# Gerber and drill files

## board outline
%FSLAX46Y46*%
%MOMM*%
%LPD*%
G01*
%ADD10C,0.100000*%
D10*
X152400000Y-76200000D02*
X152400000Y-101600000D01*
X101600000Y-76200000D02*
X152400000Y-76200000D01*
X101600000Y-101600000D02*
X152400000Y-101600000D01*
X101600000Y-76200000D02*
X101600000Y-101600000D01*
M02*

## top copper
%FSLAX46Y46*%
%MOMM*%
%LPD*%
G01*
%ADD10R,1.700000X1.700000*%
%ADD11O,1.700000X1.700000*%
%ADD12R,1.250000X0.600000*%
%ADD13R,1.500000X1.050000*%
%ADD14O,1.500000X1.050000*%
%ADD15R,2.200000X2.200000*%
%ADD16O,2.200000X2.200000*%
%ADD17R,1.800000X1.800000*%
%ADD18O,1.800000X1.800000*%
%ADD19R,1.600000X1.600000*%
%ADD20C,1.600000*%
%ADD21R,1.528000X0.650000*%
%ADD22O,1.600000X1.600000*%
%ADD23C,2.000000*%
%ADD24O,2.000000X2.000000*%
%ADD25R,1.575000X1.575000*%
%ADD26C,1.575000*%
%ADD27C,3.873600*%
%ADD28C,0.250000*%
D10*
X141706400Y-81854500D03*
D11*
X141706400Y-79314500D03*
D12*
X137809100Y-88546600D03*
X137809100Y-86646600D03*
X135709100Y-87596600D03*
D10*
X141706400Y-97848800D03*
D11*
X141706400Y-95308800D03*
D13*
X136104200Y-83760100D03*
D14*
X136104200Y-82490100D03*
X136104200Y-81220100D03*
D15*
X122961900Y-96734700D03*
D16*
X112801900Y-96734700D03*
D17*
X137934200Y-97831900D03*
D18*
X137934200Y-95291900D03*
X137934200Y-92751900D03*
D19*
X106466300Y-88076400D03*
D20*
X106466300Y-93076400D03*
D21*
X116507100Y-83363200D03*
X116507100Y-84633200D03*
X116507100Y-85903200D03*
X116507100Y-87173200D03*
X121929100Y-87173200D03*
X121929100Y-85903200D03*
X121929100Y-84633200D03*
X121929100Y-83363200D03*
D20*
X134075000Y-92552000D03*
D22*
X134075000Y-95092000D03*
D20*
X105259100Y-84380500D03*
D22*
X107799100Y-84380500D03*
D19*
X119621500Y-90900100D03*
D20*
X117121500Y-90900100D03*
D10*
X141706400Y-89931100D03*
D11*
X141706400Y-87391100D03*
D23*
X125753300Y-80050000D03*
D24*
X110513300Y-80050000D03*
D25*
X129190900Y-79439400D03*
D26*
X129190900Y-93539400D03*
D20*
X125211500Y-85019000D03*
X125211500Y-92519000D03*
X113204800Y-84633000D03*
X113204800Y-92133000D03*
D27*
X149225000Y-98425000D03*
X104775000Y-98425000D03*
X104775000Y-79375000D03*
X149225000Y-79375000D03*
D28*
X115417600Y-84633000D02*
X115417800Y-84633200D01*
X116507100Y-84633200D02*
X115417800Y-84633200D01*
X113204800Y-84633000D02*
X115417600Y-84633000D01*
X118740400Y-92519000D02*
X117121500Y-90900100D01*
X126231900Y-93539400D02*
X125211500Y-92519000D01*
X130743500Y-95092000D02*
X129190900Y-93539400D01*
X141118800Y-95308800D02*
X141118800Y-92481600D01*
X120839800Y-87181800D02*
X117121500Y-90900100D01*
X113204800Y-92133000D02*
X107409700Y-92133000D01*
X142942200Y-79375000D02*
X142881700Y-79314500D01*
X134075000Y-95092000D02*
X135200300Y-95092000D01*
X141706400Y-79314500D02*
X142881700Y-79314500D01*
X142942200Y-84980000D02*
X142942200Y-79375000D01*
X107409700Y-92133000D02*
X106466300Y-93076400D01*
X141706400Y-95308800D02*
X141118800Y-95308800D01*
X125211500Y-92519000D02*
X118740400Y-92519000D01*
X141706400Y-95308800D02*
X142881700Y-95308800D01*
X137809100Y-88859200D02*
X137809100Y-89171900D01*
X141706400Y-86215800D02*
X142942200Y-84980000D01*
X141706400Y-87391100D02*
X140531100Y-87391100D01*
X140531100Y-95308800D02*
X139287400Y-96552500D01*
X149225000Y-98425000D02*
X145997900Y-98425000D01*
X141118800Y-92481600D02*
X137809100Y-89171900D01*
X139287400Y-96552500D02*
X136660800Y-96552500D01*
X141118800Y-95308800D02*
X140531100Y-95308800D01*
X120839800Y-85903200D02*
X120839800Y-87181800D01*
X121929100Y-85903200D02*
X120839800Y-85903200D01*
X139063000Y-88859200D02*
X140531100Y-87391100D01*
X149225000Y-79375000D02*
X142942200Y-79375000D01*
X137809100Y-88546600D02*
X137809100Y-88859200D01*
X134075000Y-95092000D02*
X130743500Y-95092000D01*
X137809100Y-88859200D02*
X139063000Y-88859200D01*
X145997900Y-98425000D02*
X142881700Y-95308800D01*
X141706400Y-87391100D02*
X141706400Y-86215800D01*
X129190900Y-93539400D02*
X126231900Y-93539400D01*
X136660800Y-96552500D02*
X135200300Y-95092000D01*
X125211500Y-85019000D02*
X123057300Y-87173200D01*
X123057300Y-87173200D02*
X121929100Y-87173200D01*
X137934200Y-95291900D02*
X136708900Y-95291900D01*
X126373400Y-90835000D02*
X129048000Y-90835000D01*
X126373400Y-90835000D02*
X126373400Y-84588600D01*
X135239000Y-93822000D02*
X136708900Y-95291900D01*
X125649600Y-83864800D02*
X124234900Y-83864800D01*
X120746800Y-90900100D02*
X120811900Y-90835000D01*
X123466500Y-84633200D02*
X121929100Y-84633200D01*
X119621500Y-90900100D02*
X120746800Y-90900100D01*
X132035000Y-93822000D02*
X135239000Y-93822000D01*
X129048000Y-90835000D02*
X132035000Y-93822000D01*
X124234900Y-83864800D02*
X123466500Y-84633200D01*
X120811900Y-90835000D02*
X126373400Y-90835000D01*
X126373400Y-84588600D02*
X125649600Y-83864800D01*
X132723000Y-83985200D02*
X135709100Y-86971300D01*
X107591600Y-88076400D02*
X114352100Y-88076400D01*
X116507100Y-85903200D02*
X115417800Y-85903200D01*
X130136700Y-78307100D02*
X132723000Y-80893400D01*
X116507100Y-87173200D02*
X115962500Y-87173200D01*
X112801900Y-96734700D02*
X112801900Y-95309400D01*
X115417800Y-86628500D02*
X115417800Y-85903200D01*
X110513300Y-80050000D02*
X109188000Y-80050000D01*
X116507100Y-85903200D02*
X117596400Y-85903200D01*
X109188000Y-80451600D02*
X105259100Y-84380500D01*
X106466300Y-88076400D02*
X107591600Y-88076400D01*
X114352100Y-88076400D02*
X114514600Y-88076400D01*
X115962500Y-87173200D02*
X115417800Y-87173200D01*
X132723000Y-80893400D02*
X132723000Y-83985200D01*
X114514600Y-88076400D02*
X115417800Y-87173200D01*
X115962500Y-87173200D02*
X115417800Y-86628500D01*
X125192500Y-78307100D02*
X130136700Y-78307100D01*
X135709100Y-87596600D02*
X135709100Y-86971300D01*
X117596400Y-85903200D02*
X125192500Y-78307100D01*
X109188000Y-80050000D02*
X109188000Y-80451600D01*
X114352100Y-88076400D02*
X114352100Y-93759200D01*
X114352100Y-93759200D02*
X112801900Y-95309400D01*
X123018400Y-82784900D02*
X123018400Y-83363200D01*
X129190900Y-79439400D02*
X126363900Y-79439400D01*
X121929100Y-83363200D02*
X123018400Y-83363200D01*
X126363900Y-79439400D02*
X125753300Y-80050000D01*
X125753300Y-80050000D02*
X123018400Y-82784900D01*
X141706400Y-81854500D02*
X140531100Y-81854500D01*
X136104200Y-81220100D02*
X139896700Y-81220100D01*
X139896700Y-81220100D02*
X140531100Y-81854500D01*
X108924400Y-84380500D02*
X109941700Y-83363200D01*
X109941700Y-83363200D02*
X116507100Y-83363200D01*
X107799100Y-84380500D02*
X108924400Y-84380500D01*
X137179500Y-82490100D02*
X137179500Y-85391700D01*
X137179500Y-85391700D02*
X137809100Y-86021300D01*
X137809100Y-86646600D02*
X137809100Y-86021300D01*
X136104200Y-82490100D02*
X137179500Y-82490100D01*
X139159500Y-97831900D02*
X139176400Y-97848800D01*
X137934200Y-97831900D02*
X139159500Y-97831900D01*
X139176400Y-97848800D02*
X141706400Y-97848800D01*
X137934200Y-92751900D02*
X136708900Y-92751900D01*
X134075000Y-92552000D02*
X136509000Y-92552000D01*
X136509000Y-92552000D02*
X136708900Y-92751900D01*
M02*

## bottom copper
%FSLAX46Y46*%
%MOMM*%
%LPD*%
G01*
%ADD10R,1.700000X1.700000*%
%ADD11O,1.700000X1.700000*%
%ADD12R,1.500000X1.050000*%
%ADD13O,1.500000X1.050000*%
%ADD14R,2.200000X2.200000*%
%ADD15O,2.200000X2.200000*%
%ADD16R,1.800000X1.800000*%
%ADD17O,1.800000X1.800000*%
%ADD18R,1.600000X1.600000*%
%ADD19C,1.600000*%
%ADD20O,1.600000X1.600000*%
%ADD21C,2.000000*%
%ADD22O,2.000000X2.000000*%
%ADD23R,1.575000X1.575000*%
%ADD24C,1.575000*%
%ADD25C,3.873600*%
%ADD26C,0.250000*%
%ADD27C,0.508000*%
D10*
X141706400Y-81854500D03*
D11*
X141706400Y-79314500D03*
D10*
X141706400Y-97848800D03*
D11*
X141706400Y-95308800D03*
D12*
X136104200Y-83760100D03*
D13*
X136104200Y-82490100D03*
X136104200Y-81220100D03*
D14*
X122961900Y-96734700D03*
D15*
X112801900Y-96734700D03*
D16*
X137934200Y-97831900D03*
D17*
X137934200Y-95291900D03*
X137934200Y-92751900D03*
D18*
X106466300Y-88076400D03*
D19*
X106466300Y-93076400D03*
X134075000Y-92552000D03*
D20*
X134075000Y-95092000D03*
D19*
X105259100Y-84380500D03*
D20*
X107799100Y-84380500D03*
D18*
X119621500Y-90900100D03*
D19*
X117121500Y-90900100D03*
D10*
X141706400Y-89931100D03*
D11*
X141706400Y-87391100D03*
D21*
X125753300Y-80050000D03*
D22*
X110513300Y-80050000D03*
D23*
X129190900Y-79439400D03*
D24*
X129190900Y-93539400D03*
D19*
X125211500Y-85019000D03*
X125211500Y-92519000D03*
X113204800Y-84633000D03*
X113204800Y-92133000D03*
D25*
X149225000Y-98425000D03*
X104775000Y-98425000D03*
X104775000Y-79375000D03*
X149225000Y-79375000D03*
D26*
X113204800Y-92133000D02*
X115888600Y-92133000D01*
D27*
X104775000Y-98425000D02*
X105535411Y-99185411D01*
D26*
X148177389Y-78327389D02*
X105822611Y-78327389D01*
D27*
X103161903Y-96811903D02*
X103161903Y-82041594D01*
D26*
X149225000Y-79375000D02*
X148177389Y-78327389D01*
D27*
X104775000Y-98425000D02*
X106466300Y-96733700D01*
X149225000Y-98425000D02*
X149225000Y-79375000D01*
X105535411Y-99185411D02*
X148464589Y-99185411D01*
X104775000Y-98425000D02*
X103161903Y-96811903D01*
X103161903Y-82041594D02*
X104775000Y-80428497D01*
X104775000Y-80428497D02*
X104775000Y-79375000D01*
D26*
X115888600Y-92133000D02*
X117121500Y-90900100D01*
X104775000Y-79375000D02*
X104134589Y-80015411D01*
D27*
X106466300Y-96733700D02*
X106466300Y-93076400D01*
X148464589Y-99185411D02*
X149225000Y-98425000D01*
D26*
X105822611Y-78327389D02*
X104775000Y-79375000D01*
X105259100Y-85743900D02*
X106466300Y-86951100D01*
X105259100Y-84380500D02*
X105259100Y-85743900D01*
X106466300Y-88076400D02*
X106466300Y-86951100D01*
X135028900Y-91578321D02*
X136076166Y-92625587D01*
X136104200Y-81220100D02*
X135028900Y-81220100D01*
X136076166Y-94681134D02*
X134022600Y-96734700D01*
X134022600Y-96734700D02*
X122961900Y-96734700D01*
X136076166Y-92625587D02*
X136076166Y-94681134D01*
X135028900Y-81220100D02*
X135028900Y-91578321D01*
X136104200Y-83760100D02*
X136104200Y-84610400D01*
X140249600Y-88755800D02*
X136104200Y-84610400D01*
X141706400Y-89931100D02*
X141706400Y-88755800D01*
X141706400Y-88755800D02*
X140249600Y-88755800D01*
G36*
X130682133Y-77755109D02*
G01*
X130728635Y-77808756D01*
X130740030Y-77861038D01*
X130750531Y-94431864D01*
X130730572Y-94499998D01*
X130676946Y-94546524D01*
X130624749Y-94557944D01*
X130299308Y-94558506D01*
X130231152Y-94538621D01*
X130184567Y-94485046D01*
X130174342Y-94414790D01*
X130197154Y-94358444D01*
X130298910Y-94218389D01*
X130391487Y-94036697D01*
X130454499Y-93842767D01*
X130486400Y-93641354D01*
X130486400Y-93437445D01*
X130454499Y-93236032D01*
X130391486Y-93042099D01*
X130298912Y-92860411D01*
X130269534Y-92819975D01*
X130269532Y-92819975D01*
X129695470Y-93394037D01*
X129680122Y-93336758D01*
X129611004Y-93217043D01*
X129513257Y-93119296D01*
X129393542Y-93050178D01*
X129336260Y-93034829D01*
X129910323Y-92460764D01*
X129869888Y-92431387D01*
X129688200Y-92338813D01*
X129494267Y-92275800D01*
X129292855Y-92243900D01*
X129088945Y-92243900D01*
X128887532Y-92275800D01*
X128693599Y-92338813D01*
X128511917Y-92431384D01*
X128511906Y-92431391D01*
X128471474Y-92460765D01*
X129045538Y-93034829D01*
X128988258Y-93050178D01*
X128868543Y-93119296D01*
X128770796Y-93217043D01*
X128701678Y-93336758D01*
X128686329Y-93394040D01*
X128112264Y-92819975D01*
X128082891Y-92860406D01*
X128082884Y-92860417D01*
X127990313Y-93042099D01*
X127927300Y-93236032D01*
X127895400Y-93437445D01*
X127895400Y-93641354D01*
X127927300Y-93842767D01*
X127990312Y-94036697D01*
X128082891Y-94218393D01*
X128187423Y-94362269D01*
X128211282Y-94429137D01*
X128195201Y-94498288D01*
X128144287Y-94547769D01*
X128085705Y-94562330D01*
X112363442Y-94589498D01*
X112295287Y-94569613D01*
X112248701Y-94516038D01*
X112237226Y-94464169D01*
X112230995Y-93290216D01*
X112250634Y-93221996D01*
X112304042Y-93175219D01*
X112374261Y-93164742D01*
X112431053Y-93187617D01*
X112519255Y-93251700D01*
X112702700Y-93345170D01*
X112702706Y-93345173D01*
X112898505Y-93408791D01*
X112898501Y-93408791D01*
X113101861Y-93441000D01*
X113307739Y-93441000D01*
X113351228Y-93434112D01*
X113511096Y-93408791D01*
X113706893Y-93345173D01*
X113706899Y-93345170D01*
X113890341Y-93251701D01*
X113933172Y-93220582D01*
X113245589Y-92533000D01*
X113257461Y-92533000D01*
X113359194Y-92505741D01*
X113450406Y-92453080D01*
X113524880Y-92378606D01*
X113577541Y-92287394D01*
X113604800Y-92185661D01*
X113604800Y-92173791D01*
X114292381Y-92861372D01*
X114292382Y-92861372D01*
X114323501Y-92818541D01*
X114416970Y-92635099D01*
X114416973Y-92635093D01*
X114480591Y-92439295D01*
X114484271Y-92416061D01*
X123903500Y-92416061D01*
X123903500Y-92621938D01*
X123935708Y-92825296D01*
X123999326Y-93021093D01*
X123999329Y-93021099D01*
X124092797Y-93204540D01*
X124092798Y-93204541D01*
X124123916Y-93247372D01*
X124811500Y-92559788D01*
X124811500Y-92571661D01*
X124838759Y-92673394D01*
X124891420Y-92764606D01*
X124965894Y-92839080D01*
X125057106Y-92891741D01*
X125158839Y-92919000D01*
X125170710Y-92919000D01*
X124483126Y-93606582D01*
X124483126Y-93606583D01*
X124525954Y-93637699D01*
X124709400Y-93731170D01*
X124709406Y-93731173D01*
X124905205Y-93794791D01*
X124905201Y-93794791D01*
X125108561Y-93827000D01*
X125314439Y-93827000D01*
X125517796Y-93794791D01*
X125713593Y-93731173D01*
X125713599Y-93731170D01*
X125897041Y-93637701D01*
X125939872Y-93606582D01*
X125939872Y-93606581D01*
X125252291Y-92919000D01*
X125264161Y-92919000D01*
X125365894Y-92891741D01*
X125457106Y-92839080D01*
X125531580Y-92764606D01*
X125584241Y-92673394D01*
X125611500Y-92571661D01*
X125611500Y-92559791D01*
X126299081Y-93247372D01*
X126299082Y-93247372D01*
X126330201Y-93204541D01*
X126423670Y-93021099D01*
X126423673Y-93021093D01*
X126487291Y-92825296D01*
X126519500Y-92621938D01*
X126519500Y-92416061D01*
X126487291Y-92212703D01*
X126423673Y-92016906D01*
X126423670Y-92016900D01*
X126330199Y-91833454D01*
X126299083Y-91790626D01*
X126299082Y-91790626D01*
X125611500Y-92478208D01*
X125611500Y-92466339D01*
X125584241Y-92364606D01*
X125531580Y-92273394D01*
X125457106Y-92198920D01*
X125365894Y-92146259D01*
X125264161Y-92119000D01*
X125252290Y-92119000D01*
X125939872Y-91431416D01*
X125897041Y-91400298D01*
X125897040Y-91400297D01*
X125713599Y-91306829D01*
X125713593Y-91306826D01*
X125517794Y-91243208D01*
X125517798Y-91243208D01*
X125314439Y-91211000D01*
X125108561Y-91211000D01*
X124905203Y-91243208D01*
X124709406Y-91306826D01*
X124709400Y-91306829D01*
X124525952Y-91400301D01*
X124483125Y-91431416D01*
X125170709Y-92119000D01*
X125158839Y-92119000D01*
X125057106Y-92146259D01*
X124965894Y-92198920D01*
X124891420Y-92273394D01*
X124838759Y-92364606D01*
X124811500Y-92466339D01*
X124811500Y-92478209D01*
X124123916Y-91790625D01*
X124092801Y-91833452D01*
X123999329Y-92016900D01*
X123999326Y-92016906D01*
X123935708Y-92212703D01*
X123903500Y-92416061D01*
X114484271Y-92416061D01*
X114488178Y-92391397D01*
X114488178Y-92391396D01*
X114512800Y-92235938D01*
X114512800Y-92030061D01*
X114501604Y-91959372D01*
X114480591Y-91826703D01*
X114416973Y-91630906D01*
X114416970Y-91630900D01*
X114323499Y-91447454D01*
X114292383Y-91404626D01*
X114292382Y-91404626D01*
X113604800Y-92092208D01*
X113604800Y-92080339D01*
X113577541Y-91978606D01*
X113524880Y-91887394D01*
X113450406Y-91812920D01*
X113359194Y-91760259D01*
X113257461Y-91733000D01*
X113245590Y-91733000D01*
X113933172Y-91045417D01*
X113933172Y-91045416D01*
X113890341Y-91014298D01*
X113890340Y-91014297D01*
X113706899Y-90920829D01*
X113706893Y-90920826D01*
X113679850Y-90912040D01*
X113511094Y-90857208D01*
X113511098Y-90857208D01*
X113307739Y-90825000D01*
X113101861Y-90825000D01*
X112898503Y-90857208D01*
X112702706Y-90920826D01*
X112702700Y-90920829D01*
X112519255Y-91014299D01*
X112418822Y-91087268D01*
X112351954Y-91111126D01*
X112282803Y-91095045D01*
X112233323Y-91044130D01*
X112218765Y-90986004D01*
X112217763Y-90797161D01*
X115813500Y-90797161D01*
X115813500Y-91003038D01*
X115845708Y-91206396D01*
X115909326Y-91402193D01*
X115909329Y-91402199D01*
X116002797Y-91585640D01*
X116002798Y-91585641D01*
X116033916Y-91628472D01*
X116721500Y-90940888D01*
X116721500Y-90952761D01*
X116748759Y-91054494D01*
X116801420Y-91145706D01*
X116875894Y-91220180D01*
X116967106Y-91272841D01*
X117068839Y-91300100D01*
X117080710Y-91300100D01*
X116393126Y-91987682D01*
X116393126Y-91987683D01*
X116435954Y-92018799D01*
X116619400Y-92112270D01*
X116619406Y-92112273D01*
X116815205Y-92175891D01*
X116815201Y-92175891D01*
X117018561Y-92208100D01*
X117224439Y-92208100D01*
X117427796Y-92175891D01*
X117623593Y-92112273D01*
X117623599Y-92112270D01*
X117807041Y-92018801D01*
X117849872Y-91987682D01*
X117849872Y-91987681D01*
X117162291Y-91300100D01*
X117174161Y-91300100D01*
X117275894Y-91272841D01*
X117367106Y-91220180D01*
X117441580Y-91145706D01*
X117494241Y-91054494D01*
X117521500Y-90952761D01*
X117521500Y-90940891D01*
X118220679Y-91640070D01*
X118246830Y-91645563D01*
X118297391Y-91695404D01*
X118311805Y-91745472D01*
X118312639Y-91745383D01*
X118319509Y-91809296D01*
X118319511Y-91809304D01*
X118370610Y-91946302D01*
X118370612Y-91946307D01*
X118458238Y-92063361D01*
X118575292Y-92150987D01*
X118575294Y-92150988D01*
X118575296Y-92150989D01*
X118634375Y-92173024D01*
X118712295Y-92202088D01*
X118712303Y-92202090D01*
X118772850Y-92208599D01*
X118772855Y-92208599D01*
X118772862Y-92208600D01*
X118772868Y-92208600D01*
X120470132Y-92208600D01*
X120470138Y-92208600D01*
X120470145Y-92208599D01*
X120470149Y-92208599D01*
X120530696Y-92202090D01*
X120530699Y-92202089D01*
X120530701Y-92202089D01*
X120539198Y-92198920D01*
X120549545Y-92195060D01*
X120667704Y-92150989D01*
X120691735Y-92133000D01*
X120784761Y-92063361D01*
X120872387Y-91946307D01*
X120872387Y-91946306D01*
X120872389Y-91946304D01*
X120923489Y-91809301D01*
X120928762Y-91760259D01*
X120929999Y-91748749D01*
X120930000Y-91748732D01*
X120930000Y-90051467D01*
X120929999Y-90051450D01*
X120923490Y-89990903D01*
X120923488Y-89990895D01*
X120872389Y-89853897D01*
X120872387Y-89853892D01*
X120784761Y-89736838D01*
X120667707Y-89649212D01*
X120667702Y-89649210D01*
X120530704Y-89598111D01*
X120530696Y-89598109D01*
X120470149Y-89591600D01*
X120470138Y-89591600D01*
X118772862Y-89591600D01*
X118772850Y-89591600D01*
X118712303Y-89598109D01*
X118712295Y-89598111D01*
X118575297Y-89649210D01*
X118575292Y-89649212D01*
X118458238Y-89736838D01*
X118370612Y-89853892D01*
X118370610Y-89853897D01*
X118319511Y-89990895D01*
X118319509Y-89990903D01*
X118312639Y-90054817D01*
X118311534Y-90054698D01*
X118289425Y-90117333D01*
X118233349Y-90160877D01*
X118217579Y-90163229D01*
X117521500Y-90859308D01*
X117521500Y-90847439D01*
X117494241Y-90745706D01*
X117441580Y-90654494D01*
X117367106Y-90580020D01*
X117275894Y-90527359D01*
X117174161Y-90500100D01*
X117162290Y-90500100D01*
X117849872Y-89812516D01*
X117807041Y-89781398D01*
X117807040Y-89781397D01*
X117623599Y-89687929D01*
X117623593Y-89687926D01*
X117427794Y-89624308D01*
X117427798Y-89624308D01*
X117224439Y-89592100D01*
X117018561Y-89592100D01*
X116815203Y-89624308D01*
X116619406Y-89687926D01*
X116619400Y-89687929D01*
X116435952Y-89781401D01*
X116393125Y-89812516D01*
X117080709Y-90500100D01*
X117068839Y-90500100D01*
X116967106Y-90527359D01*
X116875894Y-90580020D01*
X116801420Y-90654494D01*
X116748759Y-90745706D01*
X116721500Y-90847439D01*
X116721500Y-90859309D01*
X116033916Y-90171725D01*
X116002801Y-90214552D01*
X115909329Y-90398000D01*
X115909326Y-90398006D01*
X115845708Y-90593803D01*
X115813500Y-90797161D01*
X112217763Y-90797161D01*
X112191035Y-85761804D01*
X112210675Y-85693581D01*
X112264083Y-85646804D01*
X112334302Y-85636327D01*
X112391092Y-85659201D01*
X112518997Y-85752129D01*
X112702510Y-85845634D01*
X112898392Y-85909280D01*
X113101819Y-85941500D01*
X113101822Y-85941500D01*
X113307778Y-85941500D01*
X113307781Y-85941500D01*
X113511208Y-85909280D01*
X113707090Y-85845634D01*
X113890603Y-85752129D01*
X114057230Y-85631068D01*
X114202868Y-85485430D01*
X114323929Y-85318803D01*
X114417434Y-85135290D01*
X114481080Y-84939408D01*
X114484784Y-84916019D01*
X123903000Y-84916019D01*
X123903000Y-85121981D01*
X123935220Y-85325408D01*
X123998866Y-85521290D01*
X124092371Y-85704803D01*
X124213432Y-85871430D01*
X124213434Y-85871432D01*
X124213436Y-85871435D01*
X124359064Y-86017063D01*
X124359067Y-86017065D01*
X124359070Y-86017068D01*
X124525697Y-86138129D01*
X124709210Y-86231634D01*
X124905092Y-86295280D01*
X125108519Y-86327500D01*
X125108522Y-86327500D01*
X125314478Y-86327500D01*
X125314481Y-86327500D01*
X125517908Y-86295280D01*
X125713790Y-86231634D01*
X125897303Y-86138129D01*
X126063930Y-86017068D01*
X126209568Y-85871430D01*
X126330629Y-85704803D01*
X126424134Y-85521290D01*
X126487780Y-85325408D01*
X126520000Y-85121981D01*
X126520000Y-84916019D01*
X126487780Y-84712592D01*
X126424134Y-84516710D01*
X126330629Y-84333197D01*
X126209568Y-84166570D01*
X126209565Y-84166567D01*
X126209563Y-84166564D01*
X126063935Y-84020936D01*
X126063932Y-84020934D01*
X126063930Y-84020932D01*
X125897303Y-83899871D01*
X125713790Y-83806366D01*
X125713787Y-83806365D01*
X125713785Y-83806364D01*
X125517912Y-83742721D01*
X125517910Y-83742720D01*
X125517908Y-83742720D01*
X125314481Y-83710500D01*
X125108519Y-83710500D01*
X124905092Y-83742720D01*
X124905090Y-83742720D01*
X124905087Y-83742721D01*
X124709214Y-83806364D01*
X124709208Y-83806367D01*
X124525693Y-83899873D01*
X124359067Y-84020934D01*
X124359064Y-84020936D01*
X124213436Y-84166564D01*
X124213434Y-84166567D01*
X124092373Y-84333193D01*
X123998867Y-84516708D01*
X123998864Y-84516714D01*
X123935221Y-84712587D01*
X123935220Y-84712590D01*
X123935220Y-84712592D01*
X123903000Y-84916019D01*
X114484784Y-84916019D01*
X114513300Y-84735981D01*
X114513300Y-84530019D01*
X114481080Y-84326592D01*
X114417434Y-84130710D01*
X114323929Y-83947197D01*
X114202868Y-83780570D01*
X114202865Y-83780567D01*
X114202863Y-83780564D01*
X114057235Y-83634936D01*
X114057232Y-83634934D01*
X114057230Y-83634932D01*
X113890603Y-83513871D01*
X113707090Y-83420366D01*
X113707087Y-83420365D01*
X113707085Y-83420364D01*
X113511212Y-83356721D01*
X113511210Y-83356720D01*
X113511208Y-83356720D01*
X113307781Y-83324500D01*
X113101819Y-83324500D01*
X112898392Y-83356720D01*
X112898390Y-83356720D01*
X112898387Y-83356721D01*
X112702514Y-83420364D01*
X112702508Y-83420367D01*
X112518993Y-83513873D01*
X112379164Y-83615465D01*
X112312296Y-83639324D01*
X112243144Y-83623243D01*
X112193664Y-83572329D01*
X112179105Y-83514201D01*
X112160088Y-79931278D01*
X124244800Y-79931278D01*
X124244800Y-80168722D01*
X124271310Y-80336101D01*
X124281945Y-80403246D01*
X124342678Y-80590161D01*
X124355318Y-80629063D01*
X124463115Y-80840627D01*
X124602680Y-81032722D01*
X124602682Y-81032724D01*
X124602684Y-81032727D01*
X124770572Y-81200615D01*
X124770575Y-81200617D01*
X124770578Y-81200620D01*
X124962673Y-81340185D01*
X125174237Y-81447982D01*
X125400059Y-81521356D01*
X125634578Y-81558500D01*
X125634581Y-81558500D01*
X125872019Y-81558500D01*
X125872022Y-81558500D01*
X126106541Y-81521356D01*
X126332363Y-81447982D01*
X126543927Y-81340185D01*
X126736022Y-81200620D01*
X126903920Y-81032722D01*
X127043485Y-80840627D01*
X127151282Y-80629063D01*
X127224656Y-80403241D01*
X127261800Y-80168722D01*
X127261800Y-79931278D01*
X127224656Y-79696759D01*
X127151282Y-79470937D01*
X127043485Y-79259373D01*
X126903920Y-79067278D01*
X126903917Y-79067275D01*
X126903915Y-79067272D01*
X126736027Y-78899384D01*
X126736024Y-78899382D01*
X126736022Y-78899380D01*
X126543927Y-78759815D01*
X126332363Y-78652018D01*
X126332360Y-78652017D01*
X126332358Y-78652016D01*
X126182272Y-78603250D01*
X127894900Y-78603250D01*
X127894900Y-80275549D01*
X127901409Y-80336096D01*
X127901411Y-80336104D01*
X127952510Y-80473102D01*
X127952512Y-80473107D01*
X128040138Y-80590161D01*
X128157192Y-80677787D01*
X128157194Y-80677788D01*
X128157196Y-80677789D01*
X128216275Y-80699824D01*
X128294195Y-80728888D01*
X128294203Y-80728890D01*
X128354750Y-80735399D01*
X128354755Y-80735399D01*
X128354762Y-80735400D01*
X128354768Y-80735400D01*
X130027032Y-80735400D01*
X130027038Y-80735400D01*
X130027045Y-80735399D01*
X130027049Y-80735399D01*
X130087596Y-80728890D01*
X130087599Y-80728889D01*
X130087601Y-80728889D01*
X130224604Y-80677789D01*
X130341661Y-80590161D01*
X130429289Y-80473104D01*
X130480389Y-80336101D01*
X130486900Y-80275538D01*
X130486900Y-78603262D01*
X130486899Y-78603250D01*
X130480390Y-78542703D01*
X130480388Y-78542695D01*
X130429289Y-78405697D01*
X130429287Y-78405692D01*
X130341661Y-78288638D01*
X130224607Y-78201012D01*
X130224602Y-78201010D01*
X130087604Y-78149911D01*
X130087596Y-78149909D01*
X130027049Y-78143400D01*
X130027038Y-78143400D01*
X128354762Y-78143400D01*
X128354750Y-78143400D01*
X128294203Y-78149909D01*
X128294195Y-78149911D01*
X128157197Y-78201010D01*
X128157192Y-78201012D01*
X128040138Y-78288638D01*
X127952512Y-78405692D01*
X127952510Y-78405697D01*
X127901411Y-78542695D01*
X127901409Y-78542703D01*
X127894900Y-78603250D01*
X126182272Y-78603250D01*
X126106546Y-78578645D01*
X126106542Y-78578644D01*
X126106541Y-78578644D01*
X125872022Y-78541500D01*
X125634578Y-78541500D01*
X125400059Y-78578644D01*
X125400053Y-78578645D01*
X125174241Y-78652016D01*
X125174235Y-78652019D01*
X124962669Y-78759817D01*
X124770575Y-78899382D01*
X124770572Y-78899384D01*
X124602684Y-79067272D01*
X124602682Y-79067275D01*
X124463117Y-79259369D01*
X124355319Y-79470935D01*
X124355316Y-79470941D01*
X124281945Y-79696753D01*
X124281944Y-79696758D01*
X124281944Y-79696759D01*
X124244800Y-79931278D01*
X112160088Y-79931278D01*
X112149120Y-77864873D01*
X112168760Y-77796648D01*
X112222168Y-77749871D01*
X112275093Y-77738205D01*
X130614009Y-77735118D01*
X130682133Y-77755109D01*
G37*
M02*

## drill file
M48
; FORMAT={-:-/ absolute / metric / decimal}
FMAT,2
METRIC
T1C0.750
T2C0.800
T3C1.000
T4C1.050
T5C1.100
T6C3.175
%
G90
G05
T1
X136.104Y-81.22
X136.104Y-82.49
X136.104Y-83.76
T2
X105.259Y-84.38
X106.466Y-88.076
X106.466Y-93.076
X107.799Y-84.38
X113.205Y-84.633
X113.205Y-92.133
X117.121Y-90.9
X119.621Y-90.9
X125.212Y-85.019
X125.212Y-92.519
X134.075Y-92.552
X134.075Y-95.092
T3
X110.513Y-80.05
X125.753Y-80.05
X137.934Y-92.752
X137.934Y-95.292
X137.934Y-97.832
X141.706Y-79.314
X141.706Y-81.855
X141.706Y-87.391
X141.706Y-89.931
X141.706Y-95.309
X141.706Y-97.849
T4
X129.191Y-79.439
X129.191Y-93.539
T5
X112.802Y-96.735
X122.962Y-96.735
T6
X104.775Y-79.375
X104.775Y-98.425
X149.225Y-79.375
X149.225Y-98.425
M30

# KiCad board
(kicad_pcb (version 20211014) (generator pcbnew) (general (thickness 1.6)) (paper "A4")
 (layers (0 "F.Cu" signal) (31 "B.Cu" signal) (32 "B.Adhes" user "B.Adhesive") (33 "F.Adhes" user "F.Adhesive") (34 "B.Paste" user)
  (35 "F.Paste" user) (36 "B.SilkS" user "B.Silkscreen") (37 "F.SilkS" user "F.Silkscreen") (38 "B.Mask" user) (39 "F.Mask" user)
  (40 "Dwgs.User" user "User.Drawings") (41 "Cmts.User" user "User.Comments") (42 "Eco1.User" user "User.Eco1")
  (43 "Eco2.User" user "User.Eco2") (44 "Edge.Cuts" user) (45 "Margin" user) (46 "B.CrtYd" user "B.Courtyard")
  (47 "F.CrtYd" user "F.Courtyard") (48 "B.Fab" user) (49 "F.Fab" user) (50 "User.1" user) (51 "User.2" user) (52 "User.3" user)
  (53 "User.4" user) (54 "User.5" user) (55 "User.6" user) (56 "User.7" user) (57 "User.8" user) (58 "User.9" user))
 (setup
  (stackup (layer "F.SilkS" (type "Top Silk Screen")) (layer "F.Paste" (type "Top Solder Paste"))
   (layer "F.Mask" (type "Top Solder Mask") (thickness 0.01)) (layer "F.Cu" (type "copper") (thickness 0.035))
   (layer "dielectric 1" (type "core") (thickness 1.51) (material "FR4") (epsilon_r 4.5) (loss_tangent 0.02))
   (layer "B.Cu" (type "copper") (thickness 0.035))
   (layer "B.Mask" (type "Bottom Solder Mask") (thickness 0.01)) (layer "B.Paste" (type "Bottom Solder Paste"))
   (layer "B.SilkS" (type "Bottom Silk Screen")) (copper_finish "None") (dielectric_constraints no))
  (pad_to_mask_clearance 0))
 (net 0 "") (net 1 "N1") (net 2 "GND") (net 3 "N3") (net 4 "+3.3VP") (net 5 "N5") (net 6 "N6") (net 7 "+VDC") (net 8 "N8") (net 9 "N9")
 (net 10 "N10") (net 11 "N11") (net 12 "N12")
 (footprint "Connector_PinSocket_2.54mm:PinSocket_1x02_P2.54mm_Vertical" (layer "F.Cu") (at 141.7064 81.8545 180)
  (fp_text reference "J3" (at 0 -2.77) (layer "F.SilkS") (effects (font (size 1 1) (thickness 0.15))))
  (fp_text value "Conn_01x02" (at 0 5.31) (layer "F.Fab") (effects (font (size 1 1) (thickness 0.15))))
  (pad "1" thru_hole rect locked (at 0 0 180) (size 1.7 1.7) (drill 1) (layers *.Cu *.Mask) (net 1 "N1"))
  (pad "2" thru_hole oval locked (at 0 2.54 180) (size 1.7 1.7) (drill 1) (layers *.Cu *.Mask) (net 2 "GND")))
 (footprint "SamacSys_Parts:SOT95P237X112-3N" (layer "F.Cu") (at 136.7591 87.5966 180)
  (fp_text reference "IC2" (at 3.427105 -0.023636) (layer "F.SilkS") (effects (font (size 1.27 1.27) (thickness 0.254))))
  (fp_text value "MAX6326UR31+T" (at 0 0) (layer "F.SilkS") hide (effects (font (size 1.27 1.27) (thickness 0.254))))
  (pad "1" smd rect locked (at -1.05 -0.95 270) (size 0.6 1.25) (layers "F.Cu" "F.Paste" "F.Mask") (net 2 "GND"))
  (pad "2" smd rect locked (at -1.05 0.95 270) (size 0.6 1.25) (layers "F.Cu" "F.Paste" "F.Mask") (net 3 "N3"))
  (pad "3" smd rect locked (at 1.05 0 270) (size 0.6 1.25) (layers "F.Cu" "F.Paste" "F.Mask") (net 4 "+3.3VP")))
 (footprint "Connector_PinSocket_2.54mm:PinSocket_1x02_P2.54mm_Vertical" (layer "F.Cu") (at 141.7064 97.8488 180)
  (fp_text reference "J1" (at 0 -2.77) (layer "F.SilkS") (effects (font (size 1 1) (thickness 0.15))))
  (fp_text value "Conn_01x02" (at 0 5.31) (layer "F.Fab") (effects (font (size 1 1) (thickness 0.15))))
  (pad "1" thru_hole rect locked (at 0 0 180) (size 1.7 1.7) (drill 1) (layers *.Cu *.Mask) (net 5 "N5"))
  (pad "2" thru_hole oval locked (at 0 2.54 180) (size 1.7 1.7) (drill 1) (layers *.Cu *.Mask) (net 2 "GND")))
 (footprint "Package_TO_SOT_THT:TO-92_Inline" (layer "F.Cu") (at 136.1042 83.7601 90)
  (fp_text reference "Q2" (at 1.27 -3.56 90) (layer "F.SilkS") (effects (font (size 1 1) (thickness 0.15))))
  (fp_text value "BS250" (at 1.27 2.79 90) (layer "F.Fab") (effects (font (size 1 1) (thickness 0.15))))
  (pad "1" thru_hole rect locked (at 0 0 90) (size 1.05 1.5) (drill 0.75) (layers *.Cu *.Mask) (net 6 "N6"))
  (pad "2" thru_hole oval locked (at 1.27 0 90) (size 1.05 1.5) (drill 0.75) (layers *.Cu *.Mask) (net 3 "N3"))
  (pad "3" thru_hole oval locked (at 2.54 0 90) (size 1.05 1.5) (drill 0.75) (layers *.Cu *.Mask) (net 1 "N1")))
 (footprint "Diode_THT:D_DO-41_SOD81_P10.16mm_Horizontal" (layer "F.Cu") (at 122.9619 96.7347 180)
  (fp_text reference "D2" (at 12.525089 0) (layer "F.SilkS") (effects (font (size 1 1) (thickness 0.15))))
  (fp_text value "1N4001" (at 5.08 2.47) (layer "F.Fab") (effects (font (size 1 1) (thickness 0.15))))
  (pad "1" thru_hole rect locked (at 0 0 180) (size 2.2 2.2) (drill 1.1) (layers *.Cu *.Mask) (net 1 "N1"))
  (pad "2" thru_hole oval locked (at 10.16 0 180) (size 2.2 2.2) (drill 1.1) (layers *.Cu *.Mask) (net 4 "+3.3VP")))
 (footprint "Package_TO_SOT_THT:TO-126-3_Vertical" (layer "F.Cu") (at 137.9342 97.8319 90)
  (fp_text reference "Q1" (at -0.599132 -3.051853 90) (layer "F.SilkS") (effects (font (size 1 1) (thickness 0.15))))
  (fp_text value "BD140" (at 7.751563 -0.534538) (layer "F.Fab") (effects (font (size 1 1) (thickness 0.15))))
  (pad "1" thru_hole rect locked (at 0 0 90) (size 1.8 1.8) (drill 1) (layers *.Cu *.Mask) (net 5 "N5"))
  (pad "2" thru_hole oval locked (at 2.54 0 90) (size 1.8 1.8) (drill 1) (layers *.Cu *.Mask) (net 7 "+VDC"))
  (pad "3" thru_hole oval locked (at 5.08 0 90) (size 1.8 1.8) (drill 1) (layers *.Cu *.Mask) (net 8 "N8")))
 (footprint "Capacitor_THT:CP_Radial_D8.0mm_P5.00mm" (layer "F.Cu") (at 106.4663 88.0764 -90)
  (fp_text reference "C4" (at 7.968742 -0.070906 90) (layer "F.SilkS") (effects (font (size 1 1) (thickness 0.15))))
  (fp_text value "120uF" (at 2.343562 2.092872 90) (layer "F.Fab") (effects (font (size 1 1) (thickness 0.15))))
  (pad "1" thru_hole rect locked (at 0 0 270) (size 1.6 1.6) (drill 0.8) (layers *.Cu *.Mask) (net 4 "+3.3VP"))
  (pad "2" thru_hole circle locked (at 5 0 270) (size 1.6 1.6) (drill 0.8) (layers *.Cu *.Mask) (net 2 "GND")))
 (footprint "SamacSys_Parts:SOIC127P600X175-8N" (layer "F.Cu") (at 119.2181 85.2682)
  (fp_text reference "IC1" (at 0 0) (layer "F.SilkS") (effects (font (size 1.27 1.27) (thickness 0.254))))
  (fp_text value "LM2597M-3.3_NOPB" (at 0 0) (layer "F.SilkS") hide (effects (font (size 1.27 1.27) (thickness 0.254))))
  (pad "1" smd rect locked (at -2.711 -1.905 90) (size 0.65 1.528) (layers "F.Cu" "F.Paste" "F.Mask") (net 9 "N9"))
  (pad "2" smd rect locked (at -2.711 -0.635 90) (size 0.65 1.528) (layers "F.Cu" "F.Paste" "F.Mask") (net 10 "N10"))
  (pad "3" smd rect locked (at -2.711 0.635 90) (size 0.65 1.528) (layers "F.Cu" "F.Paste" "F.Mask") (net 4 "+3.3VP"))
  (pad "4" smd rect locked (at -2.711 1.905 90) (size 0.65 1.528) (layers "F.Cu" "F.Paste" "F.Mask") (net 4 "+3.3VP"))
  (pad "5" smd rect locked (at 2.711 1.905 90) (size 0.65 1.528) (layers "F.Cu" "F.Paste" "F.Mask") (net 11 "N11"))
  (pad "6" smd rect locked (at 2.711 0.635 90) (size 0.65 1.528) (layers "F.Cu" "F.Paste" "F.Mask") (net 2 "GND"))
  (pad "7" smd rect locked (at 2.711 -0.635 90) (size 0.65 1.528) (layers "F.Cu" "F.Paste" "F.Mask") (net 7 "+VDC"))
  (pad "8" smd rect locked (at 2.711 -1.905 90) (size 0.65 1.528) (layers "F.Cu" "F.Paste" "F.Mask") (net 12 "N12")))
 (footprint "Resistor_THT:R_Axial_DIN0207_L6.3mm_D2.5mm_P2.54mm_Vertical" (layer "F.Cu") (at 134.075 92.552 -90)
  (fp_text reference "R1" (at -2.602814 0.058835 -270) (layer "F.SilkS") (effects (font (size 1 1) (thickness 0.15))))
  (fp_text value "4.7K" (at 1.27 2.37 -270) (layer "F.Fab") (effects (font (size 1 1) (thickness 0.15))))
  (pad "1" thru_hole circle locked (at 0 0 270) (size 1.6 1.6) (drill 0.8) (layers *.Cu *.Mask) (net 8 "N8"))
  (pad "2" thru_hole oval locked (at 2.54 0 270) (size 1.6 1.6) (drill 0.8) (layers *.Cu *.Mask) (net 2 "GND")))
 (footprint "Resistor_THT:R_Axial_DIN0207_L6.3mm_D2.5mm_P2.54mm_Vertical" (layer "F.Cu") (at 105.2591 84.3805)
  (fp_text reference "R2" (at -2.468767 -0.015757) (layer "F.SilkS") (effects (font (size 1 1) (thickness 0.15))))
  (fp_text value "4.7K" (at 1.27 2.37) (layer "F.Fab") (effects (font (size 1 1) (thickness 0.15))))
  (pad "1" thru_hole circle locked (at 0 0) (size 1.6 1.6) (drill 0.8) (layers *.Cu *.Mask) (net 4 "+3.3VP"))
  (pad "2" thru_hole oval locked (at 2.54 0) (size 1.6 1.6) (drill 0.8) (layers *.Cu *.Mask) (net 9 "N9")))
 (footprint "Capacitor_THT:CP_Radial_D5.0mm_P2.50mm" (layer "F.Cu") (at 119.6215 90.9001 180)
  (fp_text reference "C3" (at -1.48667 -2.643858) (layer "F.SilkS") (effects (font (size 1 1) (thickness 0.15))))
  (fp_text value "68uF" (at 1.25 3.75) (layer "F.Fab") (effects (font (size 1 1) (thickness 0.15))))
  (pad "1" thru_hole rect locked (at 0 0 180) (size 1.6 1.6) (drill 0.8) (layers *.Cu *.Mask) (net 7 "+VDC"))
  (pad "2" thru_hole circle locked (at 2.5 0 180) (size 1.6 1.6) (drill 0.8) (layers *.Cu *.Mask) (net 2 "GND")))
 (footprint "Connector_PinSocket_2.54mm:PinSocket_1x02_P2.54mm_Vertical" (layer "F.Cu") (at 141.7064 89.9311 180)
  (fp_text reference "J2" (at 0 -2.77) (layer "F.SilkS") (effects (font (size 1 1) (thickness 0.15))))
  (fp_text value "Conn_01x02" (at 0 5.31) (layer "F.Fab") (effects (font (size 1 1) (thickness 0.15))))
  (pad "1" thru_hole rect locked (at 0 0 180) (size 1.7 1.7) (drill 1) (layers *.Cu *.Mask) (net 6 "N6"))
  (pad "2" thru_hole oval locked (at 0 2.54 180) (size 1.7 1.7) (drill 1) (layers *.Cu *.Mask) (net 2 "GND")))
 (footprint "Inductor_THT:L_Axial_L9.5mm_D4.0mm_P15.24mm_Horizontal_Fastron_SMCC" (layer "F.Cu") (at 125.7533 80.05 180)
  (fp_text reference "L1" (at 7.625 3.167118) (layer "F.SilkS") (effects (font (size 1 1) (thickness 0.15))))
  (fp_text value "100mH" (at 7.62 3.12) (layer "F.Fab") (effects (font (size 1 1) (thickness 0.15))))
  (pad "1" thru_hole circle locked (at 0 0 180) (size 2 2) (drill 1) (layers *.Cu *.Mask) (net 12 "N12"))
  (pad "2" thru_hole oval locked (at 15.24 0 180) (size 2 2) (drill 1) (layers *.Cu *.Mask) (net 4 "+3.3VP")))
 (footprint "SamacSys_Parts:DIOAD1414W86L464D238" (layer "F.Cu") (at 129.1909 79.4394 -90)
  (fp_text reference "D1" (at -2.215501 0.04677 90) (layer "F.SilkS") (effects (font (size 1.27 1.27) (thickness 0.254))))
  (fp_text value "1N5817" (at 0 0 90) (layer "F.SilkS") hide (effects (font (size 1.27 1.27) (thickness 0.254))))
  (pad "1" thru_hole rect locked (at 0 0 270) (size 1.575 1.575) (drill 1.05) (layers *.Cu *.Mask) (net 12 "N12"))
  (pad "2" thru_hole circle locked (at 14.1 0 270) (size 1.575 1.575) (drill 1.05) (layers *.Cu *.Mask) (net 2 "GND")))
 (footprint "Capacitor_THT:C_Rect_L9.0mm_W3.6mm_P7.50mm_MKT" (layer "F.Cu") (at 125.2115 85.019 -90)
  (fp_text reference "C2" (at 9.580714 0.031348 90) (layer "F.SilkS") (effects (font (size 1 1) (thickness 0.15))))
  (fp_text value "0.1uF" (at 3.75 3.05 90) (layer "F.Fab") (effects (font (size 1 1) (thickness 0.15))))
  (pad "1" thru_hole circle locked (at 0 0 270) (size 1.6 1.6) (drill 0.8) (layers *.Cu *.Mask) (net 11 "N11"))
  (pad "2" thru_hole circle locked (at 7.5 0 270) (size 1.6 1.6) (drill 0.8) (layers *.Cu *.Mask) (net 2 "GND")))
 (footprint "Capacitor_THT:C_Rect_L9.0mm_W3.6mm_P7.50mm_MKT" (layer "F.Cu") (at 113.2048 84.633 -90)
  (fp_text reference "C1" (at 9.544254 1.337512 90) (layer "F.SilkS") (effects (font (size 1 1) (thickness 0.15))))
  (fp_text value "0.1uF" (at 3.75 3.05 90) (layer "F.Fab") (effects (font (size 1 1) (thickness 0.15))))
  (pad "1" thru_hole circle locked (at 0 0 270) (size 1.6 1.6) (drill 0.8) (layers *.Cu *.Mask) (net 10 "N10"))
  (pad "2" thru_hole circle locked (at 7.5 0 270) (size 1.6 1.6) (drill 0.8) (layers *.Cu *.Mask) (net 2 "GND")))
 (gr_line (start 152.4 76.2) (end 152.4 101.6) (layer "Edge.Cuts") (width 0.1))
 (gr_line (start 101.6 76.2) (end 152.4 76.2) (layer "Edge.Cuts") (width 0.1))
 (gr_line (start 101.6 101.6) (end 152.4 101.6) (layer "Edge.Cuts") (width 0.1))
 (gr_line (start 101.6 76.2) (end 101.6 101.6) (layer "Edge.Cuts") (width 0.1))
 (segment (start 115.4176 84.633) (end 115.4178 84.6332) (width 0.25) (layer "F.Cu") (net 10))
 (segment (start 116.5071 84.6332) (end 115.4178 84.6332) (width 0.25) (layer "F.Cu") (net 10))
 (segment (start 113.2048 84.633) (end 115.4176 84.633) (width 0.25) (layer "F.Cu") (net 10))
 (segment (start 118.7404 92.519) (end 117.1215 90.9001) (width 0.25) (layer "F.Cu") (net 2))
 (segment (start 126.2319 93.5394) (end 125.2115 92.519) (width 0.25) (layer "F.Cu") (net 2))
 (segment (start 130.7435 95.092) (end 129.1909 93.5394) (width 0.25) (layer "F.Cu") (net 2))
 (segment (start 141.1188 95.3088) (end 141.1188 92.4816) (width 0.25) (layer "F.Cu") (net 2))
 (segment (start 120.8398 87.1818) (end 117.1215 90.9001) (width 0.25) (layer "F.Cu") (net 2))
 (segment (start 113.2048 92.133) (end 107.4097 92.133) (width 0.25) (layer "F.Cu") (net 2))
 (segment (start 142.9422 79.375) (end 142.8817 79.3145) (width 0.25) (layer "F.Cu") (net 2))
 (segment (start 134.075 95.092) (end 135.2003 95.092) (width 0.25) (layer "F.Cu") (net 2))
 (segment (start 141.7064 79.3145) (end 142.8817 79.3145) (width 0.25) (layer "F.Cu") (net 2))
 (segment (start 142.9422 84.98) (end 142.9422 79.375) (width 0.25) (layer "F.Cu") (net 2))
 (segment (start 107.4097 92.133) (end 106.4663 93.0764) (width 0.25) (layer "F.Cu") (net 2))
 (segment (start 141.7064 95.3088) (end 141.1188 95.3088) (width 0.25) (layer "F.Cu") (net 2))
 (segment (start 125.2115 92.519) (end 118.7404 92.519) (width 0.25) (layer "F.Cu") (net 2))
 (segment (start 141.7064 95.3088) (end 142.8817 95.3088) (width 0.25) (layer "F.Cu") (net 2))
 (segment (start 137.8091 88.8592) (end 137.8091 89.1719) (width 0.25) (layer "F.Cu") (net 2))
 (segment (start 141.7064 86.2158) (end 142.9422 84.98) (width 0.25) (layer "F.Cu") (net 2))
 (segment (start 141.7064 87.3911) (end 140.5311 87.3911) (width 0.25) (layer "F.Cu") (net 2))
 (segment (start 140.5311 95.3088) (end 139.2874 96.5525) (width 0.25) (layer "F.Cu") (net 2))
 (segment (start 149.225 98.425) (end 145.9979 98.425) (width 0.25) (layer "F.Cu") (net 2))
 (segment (start 141.1188 92.4816) (end 137.8091 89.1719) (width 0.25) (layer "F.Cu") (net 2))
 (segment (start 139.2874 96.5525) (end 136.6608 96.5525) (width 0.25) (layer "F.Cu") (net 2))
 (segment (start 141.1188 95.3088) (end 140.5311 95.3088) (width 0.25) (layer "F.Cu") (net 2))
 (segment (start 120.8398 85.9032) (end 120.8398 87.1818) (width 0.25) (layer "F.Cu") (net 2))
 (segment (start 121.9291 85.9032) (end 120.8398 85.9032) (width 0.25) (layer "F.Cu") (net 2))
 (segment (start 139.063 88.8592) (end 140.5311 87.3911) (width 0.25) (layer "F.Cu") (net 2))
 (segment (start 149.225 79.375) (end 142.9422 79.375) (width 0.25) (layer "F.Cu") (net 2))
 (segment (start 137.8091 88.5466) (end 137.8091 88.8592) (width 0.25) (layer "F.Cu") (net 2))
 (segment (start 134.075 95.092) (end 130.7435 95.092) (width 0.25) (layer "F.Cu") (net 2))
 (segment (start 137.8091 88.8592) (end 139.063 88.8592) (width 0.25) (layer "F.Cu") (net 2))
 (segment (start 145.9979 98.425) (end 142.8817 95.3088) (width 0.25) (layer "F.Cu") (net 2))
 (segment (start 141.7064 87.3911) (end 141.7064 86.2158) (width 0.25) (layer "F.Cu") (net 2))
 (segment (start 129.1909 93.5394) (end 126.2319 93.5394) (width 0.25) (layer "F.Cu") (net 2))
 (segment (start 136.6608 96.5525) (end 135.2003 95.092) (width 0.25) (layer "F.Cu") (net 2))
 (via (at 149.225 98.425) (size 3.8736) (drill 3.175) (layers "F.Cu" "B.Cu") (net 2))
 (via (at 104.775 98.425) (size 3.8736) (drill 3.175) (layers "F.Cu" "B.Cu") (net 2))
 (via (at 104.775 79.375) (size 3.8736) (drill 3.175) (layers "F.Cu" "B.Cu") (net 2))
 (via (at 149.225 79.375) (size 3.8736) (drill 3.175) (layers "F.Cu" "B.Cu") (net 2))
 (segment (start 113.2048 92.133) (end 115.8886 92.133) (width 0.25) (layer "B.Cu") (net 2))
 (segment (start 104.775 98.425) (end 105.535411 99.185411) (width 0.508) (layer "B.Cu") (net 2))
 (segment (start 148.177389 78.327389) (end 105.822611 78.327389) (width 0.25) (layer "B.Cu") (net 2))
 (segment (start 103.161903 96.811903) (end 103.161903 82.041594) (width 0.508) (layer "B.Cu") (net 2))
 (segment (start 149.225 79.375) (end 148.177389 78.327389) (width 0.25) (layer "B.Cu") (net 2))
 (segment (start 104.775 98.425) (end 106.4663 96.7337) (width 0.508) (layer "B.Cu") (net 2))
 (segment (start 149.225 98.425) (end 149.225 79.375) (width 0.508) (layer "B.Cu") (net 2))
 (segment (start 105.535411 99.185411) (end 148.464589 99.185411) (width 0.508) (layer "B.Cu") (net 2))
 (segment (start 104.775 98.425) (end 103.161903 96.811903) (width 0.508) (layer "B.Cu") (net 2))
 (segment (start 103.161903 82.041594) (end 104.775 80.428497) (width 0.508) (layer "B.Cu") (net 2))
 (segment (start 104.775 80.428497) (end 104.775 79.375) (width 0.508) (layer "B.Cu") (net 2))
 (segment (start 115.8886 92.133) (end 117.1215 90.9001) (width 0.25) (layer "B.Cu") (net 2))
 (segment (start 104.775 79.375) (end 104.134589 80.015411) (width 0.25) (layer "B.Cu") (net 2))
 (segment (start 106.4663 96.7337) (end 106.4663 93.0764) (width 0.508) (layer "B.Cu") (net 2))
 (segment (start 148.464589 99.185411) (end 149.225 98.425) (width 0.508) (layer "B.Cu") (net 2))
 (segment (start 105.822611 78.327389) (end 104.775 79.375) (width 0.25) (layer "B.Cu") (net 2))
 (segment (start 125.2115 85.019) (end 123.0573 87.1732) (width 0.25) (layer "F.Cu") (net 11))
 (segment (start 123.0573 87.1732) (end 121.9291 87.1732) (width 0.25) (layer "F.Cu") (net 11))
 (segment (start 137.9342 95.2919) (end 136.7089 95.2919) (width 0.25) (layer "F.Cu") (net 7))
 (segment (start 126.3734 90.835) (end 129.048 90.835) (width 0.25) (layer "F.Cu") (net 7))
 (segment (start 126.3734 90.835) (end 126.3734 84.5886) (width 0.25) (layer "F.Cu") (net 7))
 (segment (start 135.239 93.822) (end 136.7089 95.2919) (width 0.25) (layer "F.Cu") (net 7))
 (segment (start 125.6496 83.8648) (end 124.2349 83.8648) (width 0.25) (layer "F.Cu") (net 7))
 (segment (start 120.7468 90.9001) (end 120.8119 90.835) (width 0.25) (layer "F.Cu") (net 7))
 (segment (start 123.4665 84.6332) (end 121.9291 84.6332) (width 0.25) (layer "F.Cu") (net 7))
 (segment (start 119.6215 90.9001) (end 120.7468 90.9001) (width 0.25) (layer "F.Cu") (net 7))
 (segment (start 132.035 93.822) (end 135.239 93.822) (width 0.25) (layer "F.Cu") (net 7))
 (segment (start 129.048 90.835) (end 132.035 93.822) (width 0.25) (layer "F.Cu") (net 7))
 (segment (start 124.2349 83.8648) (end 123.4665 84.6332) (width 0.25) (layer "F.Cu") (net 7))
 (segment (start 120.8119 90.835) (end 126.3734 90.835) (width 0.25) (layer "F.Cu") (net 7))
 (segment (start 126.3734 84.5886) (end 125.6496 83.8648) (width 0.25) (layer "F.Cu") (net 7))
 (segment (start 132.723 83.9852) (end 135.7091 86.9713) (width 0.25) (layer "F.Cu") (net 4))
 (segment (start 107.5916 88.0764) (end 114.3521 88.0764) (width 0.25) (layer "F.Cu") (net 4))
 (segment (start 116.5071 85.9032) (end 115.4178 85.9032) (width 0.25) (layer "F.Cu") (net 4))
 (segment (start 130.1367 78.3071) (end 132.723 80.8934) (width 0.25) (layer "F.Cu") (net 4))
 (segment (start 116.5071 87.1732) (end 115.9625 87.1732) (width 0.25) (layer "F.Cu") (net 4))
 (segment (start 112.8019 96.7347) (end 112.8019 95.3094) (width 0.25) (layer "F.Cu") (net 4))
 (segment (start 115.4178 86.6285) (end 115.4178 85.9032) (width 0.25) (layer "F.Cu") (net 4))
 (segment (start 110.5133 80.05) (end 109.188 80.05) (width 0.25) (layer "F.Cu") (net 4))
 (segment (start 116.5071 85.9032) (end 117.5964 85.9032) (width 0.25) (layer "F.Cu") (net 4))
 (segment (start 109.188 80.4516) (end 105.2591 84.3805) (width 0.25) (layer "F.Cu") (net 4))
 (segment (start 106.4663 88.0764) (end 107.5916 88.0764) (width 0.25) (layer "F.Cu") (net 4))
 (segment (start 114.3521 88.0764) (end 114.5146 88.0764) (width 0.25) (layer "F.Cu") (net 4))
 (segment (start 115.9625 87.1732) (end 115.4178 87.1732) (width 0.25) (layer "F.Cu") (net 4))
 (segment (start 132.723 80.8934) (end 132.723 83.9852) (width 0.25) (layer "F.Cu") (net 4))
 (segment (start 114.5146 88.0764) (end 115.4178 87.1732) (width 0.25) (layer "F.Cu") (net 4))
 (segment (start 115.9625 87.1732) (end 115.4178 86.6285) (width 0.25) (layer "F.Cu") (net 4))
 (segment (start 125.1925 78.3071) (end 130.1367 78.3071) (width 0.25) (layer "F.Cu") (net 4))
 (segment (start 135.7091 87.5966) (end 135.7091 86.9713) (width 0.25) (layer "F.Cu") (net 4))
 (segment (start 117.5964 85.9032) (end 125.1925 78.3071) (width 0.25) (layer "F.Cu") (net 4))
 (segment (start 109.188 80.05) (end 109.188 80.4516) (width 0.25) (layer "F.Cu") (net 4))
 (segment (start 114.3521 88.0764) (end 114.3521 93.7592) (width 0.25) (layer "F.Cu") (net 4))
 (segment (start 114.3521 93.7592) (end 112.8019 95.3094) (width 0.25) (layer "F.Cu") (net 4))
 (segment (start 105.2591 85.7439) (end 106.4663 86.9511) (width 0.25) (layer "B.Cu") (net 4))
 (segment (start 105.2591 84.3805) (end 105.2591 85.7439) (width 0.25) (layer "B.Cu") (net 4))
 (segment (start 106.4663 88.0764) (end 106.4663 86.9511) (width 0.25) (layer "B.Cu") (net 4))
 (segment (start 123.0184 82.7849) (end 123.0184 83.3632) (width 0.25) (layer "F.Cu") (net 12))
 (segment (start 129.1909 79.4394) (end 126.3639 79.4394) (width 0.25) (layer "F.Cu") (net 12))
 (segment (start 121.9291 83.3632) (end 123.0184 83.3632) (width 0.25) (layer "F.Cu") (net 12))
 (segment (start 126.3639 79.4394) (end 125.7533 80.05) (width 0.25) (layer "F.Cu") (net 12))
 (segment (start 125.7533 80.05) (end 123.0184 82.7849) (width 0.25) (layer "F.Cu") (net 12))
 (segment (start 141.7064 81.8545) (end 140.5311 81.8545) (width 0.25) (layer "F.Cu") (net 1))
 (segment (start 136.1042 81.2201) (end 139.8967 81.2201) (width 0.25) (layer "F.Cu") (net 1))
 (segment (start 139.8967 81.2201) (end 140.5311 81.8545) (width 0.25) (layer "F.Cu") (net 1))
 (segment (start 135.0289 91.578321) (end 136.076166 92.625587) (width 0.25) (layer "B.Cu") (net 1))
 (segment (start 136.1042 81.2201) (end 135.0289 81.2201) (width 0.25) (layer "B.Cu") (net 1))
 (segment (start 136.076166 94.681134) (end 134.0226 96.7347) (width 0.25) (layer "B.Cu") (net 1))
 (segment (start 134.0226 96.7347) (end 122.9619 96.7347) (width 0.25) (layer "B.Cu") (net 1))
 (segment (start 136.076166 92.625587) (end 136.076166 94.681134) (width 0.25) (layer "B.Cu") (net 1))
 (segment (start 135.0289 81.2201) (end 135.0289 91.578321) (width 0.25) (layer "B.Cu") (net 1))
 (segment (start 108.9244 84.3805) (end 109.9417 83.3632) (width 0.25) (layer "F.Cu") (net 9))
 (segment (start 109.9417 83.3632) (end 116.5071 83.3632) (width 0.25) (layer "F.Cu") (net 9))
 (segment (start 107.7991 84.3805) (end 108.9244 84.3805) (width 0.25) (layer "F.Cu") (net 9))
 (segment (start 137.1795 82.4901) (end 137.1795 85.3917) (width 0.25) (layer "F.Cu") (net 3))
 (segment (start 137.1795 85.3917) (end 137.8091 86.0213) (width 0.25) (layer "F.Cu") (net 3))
 (segment (start 137.8091 86.6466) (end 137.8091 86.0213) (width 0.25) (layer "F.Cu") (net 3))
 (segment (start 136.1042 82.4901) (end 137.1795 82.4901) (width 0.25) (layer "F.Cu") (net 3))
 (segment (start 139.1595 97.8319) (end 139.1764 97.8488) (width 0.25) (layer "F.Cu") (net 5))
 (segment (start 137.9342 97.8319) (end 139.1595 97.8319) (width 0.25) (layer "F.Cu") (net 5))
 (segment (start 139.1764 97.8488) (end 141.7064 97.8488) (width 0.25) (layer "F.Cu") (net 5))
 (segment (start 136.1042 83.7601) (end 136.1042 84.6104) (width 0.25) (layer "B.Cu") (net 6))
 (segment (start 140.2496 88.7558) (end 136.1042 84.6104) (width 0.25) (layer "B.Cu") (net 6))
 (segment (start 141.7064 89.9311) (end 141.7064 88.7558) (width 0.25) (layer "B.Cu") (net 6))
 (segment (start 141.7064 88.7558) (end 140.2496 88.7558) (width 0.25) (layer "B.Cu") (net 6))
 (segment (start 137.9342 92.7519) (end 136.7089 92.7519) (width 0.25) (layer "F.Cu") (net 8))
 (segment (start 134.075 92.552) (end 136.509 92.552) (width 0.25) (layer "F.Cu") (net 8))
 (segment (start 136.509 92.552) (end 136.7089 92.7519) (width 0.25) (layer "F.Cu") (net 8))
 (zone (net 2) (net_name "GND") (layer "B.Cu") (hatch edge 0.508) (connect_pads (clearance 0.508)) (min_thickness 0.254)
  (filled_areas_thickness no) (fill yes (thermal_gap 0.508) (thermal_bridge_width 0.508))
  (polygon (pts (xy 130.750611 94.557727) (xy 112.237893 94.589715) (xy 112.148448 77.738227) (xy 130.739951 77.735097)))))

